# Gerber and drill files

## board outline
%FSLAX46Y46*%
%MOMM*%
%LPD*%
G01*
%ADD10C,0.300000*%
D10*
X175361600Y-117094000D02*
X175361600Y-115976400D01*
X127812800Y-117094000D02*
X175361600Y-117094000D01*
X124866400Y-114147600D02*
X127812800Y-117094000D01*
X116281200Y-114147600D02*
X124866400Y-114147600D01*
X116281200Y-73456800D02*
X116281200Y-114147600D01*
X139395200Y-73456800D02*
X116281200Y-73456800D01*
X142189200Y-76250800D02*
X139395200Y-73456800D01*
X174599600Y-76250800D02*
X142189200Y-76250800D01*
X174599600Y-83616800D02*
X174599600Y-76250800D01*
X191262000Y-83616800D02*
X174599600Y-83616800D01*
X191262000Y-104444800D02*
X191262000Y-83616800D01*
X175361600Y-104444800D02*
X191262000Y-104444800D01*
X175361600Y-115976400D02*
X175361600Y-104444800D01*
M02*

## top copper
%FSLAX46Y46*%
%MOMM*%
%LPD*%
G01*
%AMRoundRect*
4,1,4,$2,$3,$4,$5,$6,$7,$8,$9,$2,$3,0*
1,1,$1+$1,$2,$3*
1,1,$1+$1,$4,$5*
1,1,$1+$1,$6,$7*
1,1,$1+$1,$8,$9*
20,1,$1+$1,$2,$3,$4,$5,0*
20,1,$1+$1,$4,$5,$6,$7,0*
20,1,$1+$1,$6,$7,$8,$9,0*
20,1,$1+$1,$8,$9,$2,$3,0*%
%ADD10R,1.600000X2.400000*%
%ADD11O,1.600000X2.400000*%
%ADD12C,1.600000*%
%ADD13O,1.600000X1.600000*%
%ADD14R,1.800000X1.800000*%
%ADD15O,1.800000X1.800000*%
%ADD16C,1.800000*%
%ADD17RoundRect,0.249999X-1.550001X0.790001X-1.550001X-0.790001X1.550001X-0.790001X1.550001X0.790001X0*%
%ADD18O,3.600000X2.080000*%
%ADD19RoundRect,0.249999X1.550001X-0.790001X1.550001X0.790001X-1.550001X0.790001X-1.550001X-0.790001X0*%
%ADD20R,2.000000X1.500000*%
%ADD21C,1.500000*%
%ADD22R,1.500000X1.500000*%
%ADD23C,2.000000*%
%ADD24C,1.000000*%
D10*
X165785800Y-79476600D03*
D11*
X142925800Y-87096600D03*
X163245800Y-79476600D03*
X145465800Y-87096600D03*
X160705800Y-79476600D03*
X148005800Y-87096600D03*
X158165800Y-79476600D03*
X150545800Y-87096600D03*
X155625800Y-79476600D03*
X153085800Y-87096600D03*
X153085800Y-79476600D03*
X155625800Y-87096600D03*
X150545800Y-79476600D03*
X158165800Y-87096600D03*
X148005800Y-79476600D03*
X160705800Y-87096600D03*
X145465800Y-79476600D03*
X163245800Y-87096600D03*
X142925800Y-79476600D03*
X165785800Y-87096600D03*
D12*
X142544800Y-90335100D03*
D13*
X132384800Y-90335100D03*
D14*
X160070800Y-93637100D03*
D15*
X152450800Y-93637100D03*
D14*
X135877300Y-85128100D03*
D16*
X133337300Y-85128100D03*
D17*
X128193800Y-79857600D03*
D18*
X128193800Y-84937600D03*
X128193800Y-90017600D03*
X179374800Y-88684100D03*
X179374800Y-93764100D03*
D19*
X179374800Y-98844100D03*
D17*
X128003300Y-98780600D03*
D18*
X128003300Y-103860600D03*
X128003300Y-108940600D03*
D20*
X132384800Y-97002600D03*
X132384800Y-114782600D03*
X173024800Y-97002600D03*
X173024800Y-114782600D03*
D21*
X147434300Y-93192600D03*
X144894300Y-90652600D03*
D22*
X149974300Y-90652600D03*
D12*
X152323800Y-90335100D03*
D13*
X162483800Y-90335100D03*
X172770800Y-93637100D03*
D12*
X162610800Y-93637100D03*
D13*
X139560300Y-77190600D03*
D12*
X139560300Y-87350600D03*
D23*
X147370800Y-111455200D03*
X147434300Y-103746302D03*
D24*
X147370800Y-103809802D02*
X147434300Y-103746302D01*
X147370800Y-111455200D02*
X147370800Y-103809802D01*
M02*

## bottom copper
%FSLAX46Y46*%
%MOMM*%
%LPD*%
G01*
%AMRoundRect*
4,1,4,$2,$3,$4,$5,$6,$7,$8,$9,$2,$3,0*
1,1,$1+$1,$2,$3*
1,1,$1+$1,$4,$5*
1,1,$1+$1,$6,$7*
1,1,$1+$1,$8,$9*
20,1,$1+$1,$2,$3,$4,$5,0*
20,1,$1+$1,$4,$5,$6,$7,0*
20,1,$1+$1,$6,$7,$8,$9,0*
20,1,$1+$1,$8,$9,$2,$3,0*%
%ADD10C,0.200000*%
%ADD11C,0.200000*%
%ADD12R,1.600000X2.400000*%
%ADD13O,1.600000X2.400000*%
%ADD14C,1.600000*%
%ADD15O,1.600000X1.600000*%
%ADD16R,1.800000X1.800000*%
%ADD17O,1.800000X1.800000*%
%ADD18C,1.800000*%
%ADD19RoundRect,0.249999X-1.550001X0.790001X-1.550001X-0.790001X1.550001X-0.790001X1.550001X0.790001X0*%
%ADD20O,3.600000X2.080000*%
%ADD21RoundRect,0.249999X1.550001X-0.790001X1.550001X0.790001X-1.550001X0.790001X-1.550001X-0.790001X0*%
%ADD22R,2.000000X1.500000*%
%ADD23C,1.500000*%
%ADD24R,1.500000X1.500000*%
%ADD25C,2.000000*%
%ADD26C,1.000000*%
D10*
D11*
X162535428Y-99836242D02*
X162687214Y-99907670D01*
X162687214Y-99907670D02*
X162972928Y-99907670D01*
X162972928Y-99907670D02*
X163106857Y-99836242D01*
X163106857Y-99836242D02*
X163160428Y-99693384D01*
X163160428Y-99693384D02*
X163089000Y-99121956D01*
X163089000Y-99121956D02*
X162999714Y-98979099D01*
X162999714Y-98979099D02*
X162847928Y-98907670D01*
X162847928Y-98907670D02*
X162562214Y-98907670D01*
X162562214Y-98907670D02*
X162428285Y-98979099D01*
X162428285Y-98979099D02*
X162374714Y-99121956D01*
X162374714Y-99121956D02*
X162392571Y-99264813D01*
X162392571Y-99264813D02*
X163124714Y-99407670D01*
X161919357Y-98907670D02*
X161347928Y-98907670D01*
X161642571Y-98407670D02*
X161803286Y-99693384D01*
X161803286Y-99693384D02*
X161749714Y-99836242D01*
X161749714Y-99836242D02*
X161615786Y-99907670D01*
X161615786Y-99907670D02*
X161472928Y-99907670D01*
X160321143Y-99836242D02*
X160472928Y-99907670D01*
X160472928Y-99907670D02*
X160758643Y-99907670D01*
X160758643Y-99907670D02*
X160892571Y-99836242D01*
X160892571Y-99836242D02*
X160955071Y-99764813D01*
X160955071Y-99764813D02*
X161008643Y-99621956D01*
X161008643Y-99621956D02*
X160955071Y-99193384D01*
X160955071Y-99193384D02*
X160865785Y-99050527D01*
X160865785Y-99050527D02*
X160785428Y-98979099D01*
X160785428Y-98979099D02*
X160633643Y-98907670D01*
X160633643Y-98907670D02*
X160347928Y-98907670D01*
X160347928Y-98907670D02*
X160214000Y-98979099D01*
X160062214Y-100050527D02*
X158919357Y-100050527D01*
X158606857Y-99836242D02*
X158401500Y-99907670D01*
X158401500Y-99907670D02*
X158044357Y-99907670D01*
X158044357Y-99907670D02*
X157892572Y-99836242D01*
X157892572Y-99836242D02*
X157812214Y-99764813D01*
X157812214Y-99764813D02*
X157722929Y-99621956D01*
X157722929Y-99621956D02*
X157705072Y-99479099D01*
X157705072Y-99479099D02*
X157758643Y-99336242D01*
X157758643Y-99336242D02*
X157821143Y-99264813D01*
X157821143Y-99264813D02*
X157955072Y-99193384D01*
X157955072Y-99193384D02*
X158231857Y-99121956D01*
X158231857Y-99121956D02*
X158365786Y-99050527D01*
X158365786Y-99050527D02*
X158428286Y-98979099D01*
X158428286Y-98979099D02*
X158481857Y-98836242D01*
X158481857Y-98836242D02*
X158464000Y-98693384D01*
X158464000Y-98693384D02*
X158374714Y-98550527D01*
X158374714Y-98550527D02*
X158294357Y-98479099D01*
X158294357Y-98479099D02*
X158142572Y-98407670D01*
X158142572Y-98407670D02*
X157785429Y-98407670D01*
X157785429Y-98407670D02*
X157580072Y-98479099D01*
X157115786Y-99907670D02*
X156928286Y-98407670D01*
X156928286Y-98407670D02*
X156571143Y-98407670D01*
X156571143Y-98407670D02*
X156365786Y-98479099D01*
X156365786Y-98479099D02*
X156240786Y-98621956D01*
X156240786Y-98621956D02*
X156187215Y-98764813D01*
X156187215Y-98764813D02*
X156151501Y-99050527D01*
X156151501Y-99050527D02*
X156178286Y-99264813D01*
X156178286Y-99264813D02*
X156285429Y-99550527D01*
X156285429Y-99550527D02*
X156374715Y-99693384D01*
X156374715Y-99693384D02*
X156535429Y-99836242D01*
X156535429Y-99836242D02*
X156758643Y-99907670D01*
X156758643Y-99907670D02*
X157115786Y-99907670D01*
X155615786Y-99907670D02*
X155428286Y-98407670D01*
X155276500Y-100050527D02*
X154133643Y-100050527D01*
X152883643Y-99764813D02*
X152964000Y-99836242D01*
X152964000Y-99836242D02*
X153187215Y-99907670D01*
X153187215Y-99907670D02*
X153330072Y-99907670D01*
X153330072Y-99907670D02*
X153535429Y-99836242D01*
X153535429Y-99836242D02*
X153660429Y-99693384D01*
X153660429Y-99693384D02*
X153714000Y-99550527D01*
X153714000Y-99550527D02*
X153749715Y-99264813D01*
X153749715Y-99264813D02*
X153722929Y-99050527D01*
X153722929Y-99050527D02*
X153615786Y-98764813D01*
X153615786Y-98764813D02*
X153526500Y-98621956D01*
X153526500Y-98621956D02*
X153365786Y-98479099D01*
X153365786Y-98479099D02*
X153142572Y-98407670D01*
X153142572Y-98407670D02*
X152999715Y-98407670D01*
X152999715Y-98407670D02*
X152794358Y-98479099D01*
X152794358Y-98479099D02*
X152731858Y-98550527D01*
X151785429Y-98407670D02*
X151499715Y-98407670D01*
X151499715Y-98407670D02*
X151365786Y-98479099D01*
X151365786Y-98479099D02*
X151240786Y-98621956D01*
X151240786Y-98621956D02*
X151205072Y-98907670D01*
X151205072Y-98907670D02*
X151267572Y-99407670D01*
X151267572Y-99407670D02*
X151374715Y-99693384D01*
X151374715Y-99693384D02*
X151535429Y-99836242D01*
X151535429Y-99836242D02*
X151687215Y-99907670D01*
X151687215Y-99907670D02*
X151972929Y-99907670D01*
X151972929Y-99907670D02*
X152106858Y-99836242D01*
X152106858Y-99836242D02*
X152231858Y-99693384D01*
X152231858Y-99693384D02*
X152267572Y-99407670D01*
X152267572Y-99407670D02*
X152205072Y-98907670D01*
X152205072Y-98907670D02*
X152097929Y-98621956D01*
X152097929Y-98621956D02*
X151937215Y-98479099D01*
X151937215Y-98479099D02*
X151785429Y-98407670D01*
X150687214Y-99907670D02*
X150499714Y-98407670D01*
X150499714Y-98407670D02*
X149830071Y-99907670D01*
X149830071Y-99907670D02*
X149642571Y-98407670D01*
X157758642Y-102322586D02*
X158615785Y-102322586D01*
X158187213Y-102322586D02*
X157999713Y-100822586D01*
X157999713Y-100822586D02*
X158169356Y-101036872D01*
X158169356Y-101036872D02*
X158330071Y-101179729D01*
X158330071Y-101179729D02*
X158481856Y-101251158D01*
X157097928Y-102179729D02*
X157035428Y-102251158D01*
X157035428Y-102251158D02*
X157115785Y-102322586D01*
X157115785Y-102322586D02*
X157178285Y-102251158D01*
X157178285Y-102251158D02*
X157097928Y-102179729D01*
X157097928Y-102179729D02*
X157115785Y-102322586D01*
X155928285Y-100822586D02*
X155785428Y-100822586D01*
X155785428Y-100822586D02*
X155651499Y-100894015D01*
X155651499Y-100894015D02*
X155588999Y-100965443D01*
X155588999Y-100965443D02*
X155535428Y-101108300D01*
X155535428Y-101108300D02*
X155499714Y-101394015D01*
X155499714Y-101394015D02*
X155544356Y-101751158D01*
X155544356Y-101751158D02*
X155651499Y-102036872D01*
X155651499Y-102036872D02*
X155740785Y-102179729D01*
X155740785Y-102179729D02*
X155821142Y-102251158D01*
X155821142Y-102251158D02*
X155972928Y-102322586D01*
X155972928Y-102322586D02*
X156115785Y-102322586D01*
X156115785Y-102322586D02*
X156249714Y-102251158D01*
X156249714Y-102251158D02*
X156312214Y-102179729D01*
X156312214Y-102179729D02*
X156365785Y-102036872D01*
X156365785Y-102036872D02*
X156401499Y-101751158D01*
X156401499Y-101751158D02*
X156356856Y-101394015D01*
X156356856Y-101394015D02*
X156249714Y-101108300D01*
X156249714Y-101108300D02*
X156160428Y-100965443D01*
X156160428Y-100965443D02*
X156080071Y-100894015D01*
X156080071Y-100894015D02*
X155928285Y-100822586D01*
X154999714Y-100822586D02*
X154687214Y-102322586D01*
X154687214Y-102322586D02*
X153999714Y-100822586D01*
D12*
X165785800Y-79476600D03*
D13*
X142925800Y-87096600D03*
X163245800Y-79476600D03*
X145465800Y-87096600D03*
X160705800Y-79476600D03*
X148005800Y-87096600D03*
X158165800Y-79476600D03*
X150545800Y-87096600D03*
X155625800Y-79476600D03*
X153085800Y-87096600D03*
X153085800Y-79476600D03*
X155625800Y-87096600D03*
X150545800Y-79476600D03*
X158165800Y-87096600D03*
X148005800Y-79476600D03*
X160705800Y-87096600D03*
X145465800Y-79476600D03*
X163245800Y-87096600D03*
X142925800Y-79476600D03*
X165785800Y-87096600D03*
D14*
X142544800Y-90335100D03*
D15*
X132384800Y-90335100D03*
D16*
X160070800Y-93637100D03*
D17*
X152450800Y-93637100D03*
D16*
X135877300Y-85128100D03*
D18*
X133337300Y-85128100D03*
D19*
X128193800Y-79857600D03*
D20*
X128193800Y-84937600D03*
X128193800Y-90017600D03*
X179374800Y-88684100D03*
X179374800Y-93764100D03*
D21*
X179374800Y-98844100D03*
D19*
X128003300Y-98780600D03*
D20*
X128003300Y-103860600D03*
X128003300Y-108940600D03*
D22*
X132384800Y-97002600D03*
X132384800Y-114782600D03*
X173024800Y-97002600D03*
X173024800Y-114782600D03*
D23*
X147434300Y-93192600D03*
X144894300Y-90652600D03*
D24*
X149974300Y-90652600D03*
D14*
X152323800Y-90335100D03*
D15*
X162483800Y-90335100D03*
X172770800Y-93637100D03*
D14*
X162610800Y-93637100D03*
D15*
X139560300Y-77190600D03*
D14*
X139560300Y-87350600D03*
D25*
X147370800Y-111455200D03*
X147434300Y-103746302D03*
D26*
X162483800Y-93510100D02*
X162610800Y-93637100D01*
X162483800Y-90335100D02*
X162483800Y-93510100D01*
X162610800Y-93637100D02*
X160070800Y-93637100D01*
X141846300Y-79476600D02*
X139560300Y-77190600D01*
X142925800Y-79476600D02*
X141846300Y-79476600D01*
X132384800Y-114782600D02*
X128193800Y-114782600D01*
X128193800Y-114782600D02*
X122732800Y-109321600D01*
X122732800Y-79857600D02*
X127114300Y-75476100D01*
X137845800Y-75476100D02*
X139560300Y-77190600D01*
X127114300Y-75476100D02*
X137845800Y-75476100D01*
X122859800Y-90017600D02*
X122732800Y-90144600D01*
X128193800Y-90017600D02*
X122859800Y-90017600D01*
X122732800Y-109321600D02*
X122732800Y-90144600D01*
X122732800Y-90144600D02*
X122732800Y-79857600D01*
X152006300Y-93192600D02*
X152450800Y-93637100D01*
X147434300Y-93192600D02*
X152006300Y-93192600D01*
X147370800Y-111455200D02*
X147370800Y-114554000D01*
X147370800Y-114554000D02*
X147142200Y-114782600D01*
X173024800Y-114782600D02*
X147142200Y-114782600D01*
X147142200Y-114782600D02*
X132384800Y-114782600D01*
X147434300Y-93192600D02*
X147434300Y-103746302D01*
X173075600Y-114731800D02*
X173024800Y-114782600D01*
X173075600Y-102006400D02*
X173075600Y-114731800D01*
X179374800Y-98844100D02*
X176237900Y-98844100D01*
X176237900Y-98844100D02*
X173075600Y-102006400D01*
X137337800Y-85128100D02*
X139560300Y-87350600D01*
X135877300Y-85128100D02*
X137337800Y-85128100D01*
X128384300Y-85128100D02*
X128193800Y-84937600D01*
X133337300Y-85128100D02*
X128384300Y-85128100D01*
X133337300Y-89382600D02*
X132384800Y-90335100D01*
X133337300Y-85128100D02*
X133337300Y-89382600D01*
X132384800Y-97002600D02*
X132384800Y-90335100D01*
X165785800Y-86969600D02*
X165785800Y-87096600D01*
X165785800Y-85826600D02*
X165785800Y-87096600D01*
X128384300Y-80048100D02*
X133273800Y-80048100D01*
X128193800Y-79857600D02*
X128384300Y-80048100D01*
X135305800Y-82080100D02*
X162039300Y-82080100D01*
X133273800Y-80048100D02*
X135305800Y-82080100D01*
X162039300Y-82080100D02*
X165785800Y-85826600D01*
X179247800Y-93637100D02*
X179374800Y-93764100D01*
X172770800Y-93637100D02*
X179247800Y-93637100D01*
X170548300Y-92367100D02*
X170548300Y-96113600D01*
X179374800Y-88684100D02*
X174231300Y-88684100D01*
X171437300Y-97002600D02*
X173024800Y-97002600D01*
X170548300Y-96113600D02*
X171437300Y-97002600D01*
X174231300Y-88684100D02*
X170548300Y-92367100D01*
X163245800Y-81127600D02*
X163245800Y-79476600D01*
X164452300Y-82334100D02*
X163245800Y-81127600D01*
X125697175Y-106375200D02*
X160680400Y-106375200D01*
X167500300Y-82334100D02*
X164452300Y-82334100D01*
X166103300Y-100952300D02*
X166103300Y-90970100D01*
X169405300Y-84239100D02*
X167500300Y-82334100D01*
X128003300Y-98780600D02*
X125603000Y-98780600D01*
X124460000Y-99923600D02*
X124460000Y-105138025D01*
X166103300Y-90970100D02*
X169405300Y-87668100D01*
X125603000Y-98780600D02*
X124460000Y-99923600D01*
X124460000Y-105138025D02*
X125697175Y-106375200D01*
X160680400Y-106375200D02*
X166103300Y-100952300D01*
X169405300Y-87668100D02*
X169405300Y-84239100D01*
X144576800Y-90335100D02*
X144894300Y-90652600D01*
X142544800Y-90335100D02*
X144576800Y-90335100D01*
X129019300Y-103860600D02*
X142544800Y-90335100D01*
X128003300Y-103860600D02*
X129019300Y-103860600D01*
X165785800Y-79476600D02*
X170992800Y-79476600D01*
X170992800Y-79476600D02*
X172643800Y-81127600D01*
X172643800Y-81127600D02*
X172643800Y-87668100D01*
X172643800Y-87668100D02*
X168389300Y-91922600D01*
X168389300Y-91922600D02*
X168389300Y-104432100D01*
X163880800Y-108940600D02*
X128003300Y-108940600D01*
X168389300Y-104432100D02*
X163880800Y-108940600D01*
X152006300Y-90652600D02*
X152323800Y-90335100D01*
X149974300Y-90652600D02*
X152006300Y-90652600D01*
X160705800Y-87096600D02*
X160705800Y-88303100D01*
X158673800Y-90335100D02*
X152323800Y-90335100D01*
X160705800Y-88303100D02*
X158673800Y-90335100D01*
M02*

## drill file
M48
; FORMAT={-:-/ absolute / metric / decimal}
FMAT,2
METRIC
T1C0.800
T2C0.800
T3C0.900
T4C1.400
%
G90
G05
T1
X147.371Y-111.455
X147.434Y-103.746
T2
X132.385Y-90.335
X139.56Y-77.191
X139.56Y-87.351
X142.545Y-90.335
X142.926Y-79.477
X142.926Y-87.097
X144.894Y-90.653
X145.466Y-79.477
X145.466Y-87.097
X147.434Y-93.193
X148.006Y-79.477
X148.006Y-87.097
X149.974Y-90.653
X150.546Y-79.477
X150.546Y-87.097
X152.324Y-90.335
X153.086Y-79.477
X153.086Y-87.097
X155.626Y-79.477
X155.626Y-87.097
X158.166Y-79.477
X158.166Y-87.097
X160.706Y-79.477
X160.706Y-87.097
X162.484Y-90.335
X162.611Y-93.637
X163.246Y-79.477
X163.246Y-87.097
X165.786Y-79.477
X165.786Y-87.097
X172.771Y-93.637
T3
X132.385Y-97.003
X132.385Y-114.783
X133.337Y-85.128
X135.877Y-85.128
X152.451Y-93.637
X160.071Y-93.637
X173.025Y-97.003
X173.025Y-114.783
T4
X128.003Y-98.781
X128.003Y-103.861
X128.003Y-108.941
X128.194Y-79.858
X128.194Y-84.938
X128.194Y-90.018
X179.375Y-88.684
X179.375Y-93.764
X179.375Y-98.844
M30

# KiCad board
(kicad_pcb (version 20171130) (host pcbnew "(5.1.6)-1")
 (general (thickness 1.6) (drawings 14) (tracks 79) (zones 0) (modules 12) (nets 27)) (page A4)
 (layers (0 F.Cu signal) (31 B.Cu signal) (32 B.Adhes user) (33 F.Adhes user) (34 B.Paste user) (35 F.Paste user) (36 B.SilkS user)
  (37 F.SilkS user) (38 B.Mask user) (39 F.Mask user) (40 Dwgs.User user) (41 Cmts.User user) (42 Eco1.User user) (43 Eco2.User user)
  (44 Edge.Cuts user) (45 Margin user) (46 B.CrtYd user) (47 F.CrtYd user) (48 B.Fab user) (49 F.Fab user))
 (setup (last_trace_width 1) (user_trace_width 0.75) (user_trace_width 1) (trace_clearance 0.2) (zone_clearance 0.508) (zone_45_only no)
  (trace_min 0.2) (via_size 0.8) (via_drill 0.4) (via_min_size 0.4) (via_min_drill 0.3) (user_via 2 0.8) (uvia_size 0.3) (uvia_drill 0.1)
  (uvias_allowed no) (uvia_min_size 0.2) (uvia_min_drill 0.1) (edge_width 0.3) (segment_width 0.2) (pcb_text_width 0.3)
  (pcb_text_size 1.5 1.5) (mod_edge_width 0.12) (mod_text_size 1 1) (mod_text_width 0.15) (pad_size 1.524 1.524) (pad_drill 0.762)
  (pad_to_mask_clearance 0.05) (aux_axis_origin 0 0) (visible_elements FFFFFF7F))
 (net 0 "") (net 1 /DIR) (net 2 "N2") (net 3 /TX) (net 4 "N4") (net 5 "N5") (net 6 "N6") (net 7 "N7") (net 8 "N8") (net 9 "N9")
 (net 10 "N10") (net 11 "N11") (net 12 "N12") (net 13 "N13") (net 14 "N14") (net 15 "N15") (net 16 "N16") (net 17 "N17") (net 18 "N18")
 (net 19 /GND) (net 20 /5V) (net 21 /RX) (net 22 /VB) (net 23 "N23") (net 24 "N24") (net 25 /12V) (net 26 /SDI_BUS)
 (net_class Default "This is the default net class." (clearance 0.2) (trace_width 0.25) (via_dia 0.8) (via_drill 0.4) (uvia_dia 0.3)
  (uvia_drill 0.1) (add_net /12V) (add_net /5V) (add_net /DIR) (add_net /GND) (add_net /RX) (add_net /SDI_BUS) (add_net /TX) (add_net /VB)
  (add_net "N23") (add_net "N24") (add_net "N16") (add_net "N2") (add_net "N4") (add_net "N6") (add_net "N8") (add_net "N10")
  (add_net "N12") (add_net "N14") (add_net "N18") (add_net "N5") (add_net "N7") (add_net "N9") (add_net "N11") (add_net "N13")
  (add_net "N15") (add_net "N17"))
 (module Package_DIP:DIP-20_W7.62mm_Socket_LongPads (layer F.Cu) (at 165.7858 79.4766 270)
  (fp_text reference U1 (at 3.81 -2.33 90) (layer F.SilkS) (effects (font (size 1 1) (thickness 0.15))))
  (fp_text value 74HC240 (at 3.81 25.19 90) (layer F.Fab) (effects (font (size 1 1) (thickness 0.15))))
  (pad 1 thru_hole rect (at 0 0 270) (size 2.4 1.6) (drill 0.8) (layers *.Cu *.Mask) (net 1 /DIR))
  (pad 11 thru_hole oval (at 7.62 22.86 270) (size 2.4 1.6) (drill 0.8) (layers *.Cu *.Mask) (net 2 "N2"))
  (pad 2 thru_hole oval (at 0 2.54 270) (size 2.4 1.6) (drill 0.8) (layers *.Cu *.Mask) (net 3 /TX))
  (pad 12 thru_hole oval (at 7.62 20.32 270) (size 2.4 1.6) (drill 0.8) (layers *.Cu *.Mask) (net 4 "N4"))
  (pad 3 thru_hole oval (at 0 5.08 270) (size 2.4 1.6) (drill 0.8) (layers *.Cu *.Mask) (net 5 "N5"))
  (pad 13 thru_hole oval (at 7.62 17.78 270) (size 2.4 1.6) (drill 0.8) (layers *.Cu *.Mask) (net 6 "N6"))
  (pad 4 thru_hole oval (at 0 7.62 270) (size 2.4 1.6) (drill 0.8) (layers *.Cu *.Mask) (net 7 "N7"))
  (pad 14 thru_hole oval (at 7.62 15.24 270) (size 2.4 1.6) (drill 0.8) (layers *.Cu *.Mask) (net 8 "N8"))
  (pad 5 thru_hole oval (at 0 10.16 270) (size 2.4 1.6) (drill 0.8) (layers *.Cu *.Mask) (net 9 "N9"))
  (pad 15 thru_hole oval (at 7.62 12.7 270) (size 2.4 1.6) (drill 0.8) (layers *.Cu *.Mask) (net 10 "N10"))
  (pad 6 thru_hole oval (at 0 12.7 270) (size 2.4 1.6) (drill 0.8) (layers *.Cu *.Mask) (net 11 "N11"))
  (pad 16 thru_hole oval (at 7.62 10.16 270) (size 2.4 1.6) (drill 0.8) (layers *.Cu *.Mask) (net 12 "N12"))
  (pad 7 thru_hole oval (at 0 15.24 270) (size 2.4 1.6) (drill 0.8) (layers *.Cu *.Mask) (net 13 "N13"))
  (pad 17 thru_hole oval (at 7.62 7.62 270) (size 2.4 1.6) (drill 0.8) (layers *.Cu *.Mask) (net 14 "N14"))
  (pad 8 thru_hole oval (at 0 17.78 270) (size 2.4 1.6) (drill 0.8) (layers *.Cu *.Mask) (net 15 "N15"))
  (pad 18 thru_hole oval (at 7.62 5.08 270) (size 2.4 1.6) (drill 0.8) (layers *.Cu *.Mask) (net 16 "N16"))
  (pad 9 thru_hole oval (at 0 20.32 270) (size 2.4 1.6) (drill 0.8) (layers *.Cu *.Mask) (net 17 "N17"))
  (pad 19 thru_hole oval (at 7.62 2.54 270) (size 2.4 1.6) (drill 0.8) (layers *.Cu *.Mask) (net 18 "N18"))
  (pad 10 thru_hole oval (at 0 22.86 270) (size 2.4 1.6) (drill 0.8) (layers *.Cu *.Mask) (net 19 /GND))
  (pad 20 thru_hole oval (at 7.62 0 270) (size 2.4 1.6) (drill 0.8) (layers *.Cu *.Mask) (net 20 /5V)))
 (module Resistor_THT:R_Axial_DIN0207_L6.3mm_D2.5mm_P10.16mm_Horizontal (layer F.Cu) (at 142.5448 90.3351 180)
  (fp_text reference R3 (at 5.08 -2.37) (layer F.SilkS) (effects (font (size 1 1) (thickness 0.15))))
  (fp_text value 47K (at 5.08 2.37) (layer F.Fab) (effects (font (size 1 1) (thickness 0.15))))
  (pad 1 thru_hole circle (at 0 0 180) (size 1.6 1.6) (drill 0.8) (layers *.Cu *.Mask) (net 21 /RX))
  (pad 2 thru_hole oval (at 10.16 0 180) (size 1.6 1.6) (drill 0.8) (layers *.Cu *.Mask) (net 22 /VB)))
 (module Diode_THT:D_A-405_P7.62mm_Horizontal (layer F.Cu) (at 160.0708 93.6371 180)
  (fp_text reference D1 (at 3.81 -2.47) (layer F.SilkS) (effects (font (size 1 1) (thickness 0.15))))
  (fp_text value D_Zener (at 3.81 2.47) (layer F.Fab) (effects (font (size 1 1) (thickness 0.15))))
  (pad 1 thru_hole rect (at 0 0 180) (size 1.8 1.8) (drill 0.9) (layers *.Cu *.Mask) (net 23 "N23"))
  (pad 2 thru_hole oval (at 7.62 0 180) (size 1.8 1.8) (drill 0.9) (layers *.Cu *.Mask) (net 19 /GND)))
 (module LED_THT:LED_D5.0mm (layer F.Cu) (at 135.8773 85.1281 180)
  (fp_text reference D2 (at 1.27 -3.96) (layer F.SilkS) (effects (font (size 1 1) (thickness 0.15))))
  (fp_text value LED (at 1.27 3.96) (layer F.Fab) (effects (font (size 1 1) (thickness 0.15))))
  (pad 1 thru_hole rect (at 0 0 180) (size 1.8 1.8) (drill 0.9) (layers *.Cu *.Mask) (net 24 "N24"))
  (pad 2 thru_hole circle (at 2.54 0 180) (size 1.8 1.8) (drill 0.9) (layers *.Cu *.Mask) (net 22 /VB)))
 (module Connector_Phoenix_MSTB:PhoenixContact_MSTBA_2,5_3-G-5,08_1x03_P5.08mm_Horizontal (layer F.Cu) (at 128.1938 79.8576 270)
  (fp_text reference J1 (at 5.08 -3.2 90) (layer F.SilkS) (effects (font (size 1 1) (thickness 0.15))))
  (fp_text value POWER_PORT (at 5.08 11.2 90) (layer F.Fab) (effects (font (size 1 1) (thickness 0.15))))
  (pad 1 thru_hole roundrect (at 0 0 270) (size 2.08 3.6) (drill 1.4) (layers *.Cu *.Mask) (roundrect_rratio 0.120192) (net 20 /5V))
  (pad 2 thru_hole oval (at 5.08 0 270) (size 2.08 3.6) (drill 1.4) (layers *.Cu *.Mask) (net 22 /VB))
  (pad 3 thru_hole oval (at 10.16 0 270) (size 2.08 3.6) (drill 1.4) (layers *.Cu *.Mask) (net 19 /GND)))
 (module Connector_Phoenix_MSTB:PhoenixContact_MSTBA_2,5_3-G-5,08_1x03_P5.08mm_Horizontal (layer F.Cu) (at 179.3748 98.8441 90)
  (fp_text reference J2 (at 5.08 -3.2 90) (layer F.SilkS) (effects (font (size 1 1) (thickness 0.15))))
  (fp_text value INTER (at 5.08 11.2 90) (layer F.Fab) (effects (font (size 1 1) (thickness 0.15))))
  (pad 3 thru_hole oval (at 10.16 0 90) (size 2.08 3.6) (drill 1.4) (layers *.Cu *.Mask) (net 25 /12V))
  (pad 2 thru_hole oval (at 5.08 0 90) (size 2.08 3.6) (drill 1.4) (layers *.Cu *.Mask) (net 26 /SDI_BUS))
  (pad 1 thru_hole roundrect (at 0 0 90) (size 2.08 3.6) (drill 1.4) (layers *.Cu *.Mask) (roundrect_rratio 0.120192) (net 19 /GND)))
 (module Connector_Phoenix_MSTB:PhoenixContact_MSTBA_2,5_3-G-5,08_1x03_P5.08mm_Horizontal (layer F.Cu) (at 128.0033 98.7806 270)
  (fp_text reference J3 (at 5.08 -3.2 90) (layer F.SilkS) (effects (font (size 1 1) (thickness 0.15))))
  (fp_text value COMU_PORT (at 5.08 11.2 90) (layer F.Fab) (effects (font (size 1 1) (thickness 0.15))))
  (pad 1 thru_hole roundrect (at 0 0 270) (size 2.08 3.6) (drill 1.4) (layers *.Cu *.Mask) (roundrect_rratio 0.120192) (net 3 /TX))
  (pad 2 thru_hole oval (at 5.08 0 270) (size 2.08 3.6) (drill 1.4) (layers *.Cu *.Mask) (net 21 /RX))
  (pad 3 thru_hole oval (at 10.16 0 270) (size 2.08 3.6) (drill 1.4) (layers *.Cu *.Mask) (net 1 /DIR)))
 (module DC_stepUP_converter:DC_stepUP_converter (layer F.Cu) (at 152.7048 90.6526)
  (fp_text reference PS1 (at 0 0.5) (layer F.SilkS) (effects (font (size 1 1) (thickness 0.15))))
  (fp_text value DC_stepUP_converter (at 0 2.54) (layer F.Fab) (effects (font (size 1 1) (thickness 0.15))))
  (pad 1 thru_hole rect (at -20.32 6.35) (size 2 1.5) (drill 0.9) (layers *.Cu *.Mask) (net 22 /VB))
  (pad 2 thru_hole rect (at -20.32 24.13) (size 2 1.5) (drill 0.9) (layers *.Cu *.Mask) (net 19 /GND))
  (pad 3 thru_hole rect (at 20.32 6.35) (size 2 1.5) (drill 0.9) (layers *.Cu *.Mask) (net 25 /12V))
  (pad 4 thru_hole rect (at 20.32 24.13) (size 2 1.5) (drill 0.9) (layers *.Cu *.Mask) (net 19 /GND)))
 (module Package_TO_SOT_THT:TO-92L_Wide (layer F.Cu) (at 149.9743 90.6526 180)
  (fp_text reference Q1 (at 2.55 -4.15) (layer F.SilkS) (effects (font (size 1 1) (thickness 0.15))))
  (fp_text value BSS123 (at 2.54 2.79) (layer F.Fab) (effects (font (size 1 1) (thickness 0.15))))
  (pad 2 thru_hole circle (at 2.54 -2.54 270) (size 1.5 1.5) (drill 0.8) (layers *.Cu *.Mask) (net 19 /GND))
  (pad 3 thru_hole circle (at 5.08 0 270) (size 1.5 1.5) (drill 0.8) (layers *.Cu *.Mask) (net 21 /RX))
  (pad 1 thru_hole rect (at 0 0 270) (size 1.5 1.5) (drill 0.8) (layers *.Cu *.Mask) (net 16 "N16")))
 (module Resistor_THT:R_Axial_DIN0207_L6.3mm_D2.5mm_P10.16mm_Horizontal (layer F.Cu) (at 152.3238 90.3351)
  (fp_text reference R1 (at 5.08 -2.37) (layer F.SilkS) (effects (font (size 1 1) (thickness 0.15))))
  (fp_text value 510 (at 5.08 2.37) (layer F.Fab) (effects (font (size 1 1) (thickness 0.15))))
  (pad 1 thru_hole circle (at 0 0) (size 1.6 1.6) (drill 0.8) (layers *.Cu *.Mask) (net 16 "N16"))
  (pad 2 thru_hole oval (at 10.16 0) (size 1.6 1.6) (drill 0.8) (layers *.Cu *.Mask) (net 23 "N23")))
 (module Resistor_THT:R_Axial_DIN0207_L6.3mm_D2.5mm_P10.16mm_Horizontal (layer F.Cu) (at 162.6108 93.6371)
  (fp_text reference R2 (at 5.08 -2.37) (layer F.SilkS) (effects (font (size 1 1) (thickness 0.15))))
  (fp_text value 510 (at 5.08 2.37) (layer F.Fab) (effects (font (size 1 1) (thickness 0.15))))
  (pad 2 thru_hole oval (at 10.16 0) (size 1.6 1.6) (drill 0.8) (layers *.Cu *.Mask) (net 26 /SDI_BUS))
  (pad 1 thru_hole circle (at 0 0) (size 1.6 1.6) (drill 0.8) (layers *.Cu *.Mask) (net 23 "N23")))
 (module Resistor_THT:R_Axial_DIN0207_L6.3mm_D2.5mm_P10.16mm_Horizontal (layer F.Cu) (at 139.5603 87.3506 90)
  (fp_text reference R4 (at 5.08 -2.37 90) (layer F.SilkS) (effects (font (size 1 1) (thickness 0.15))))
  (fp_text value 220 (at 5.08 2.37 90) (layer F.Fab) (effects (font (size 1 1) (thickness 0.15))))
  (pad 2 thru_hole oval (at 10.16 0 90) (size 1.6 1.6) (drill 0.8) (layers *.Cu *.Mask) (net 19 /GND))
  (pad 1 thru_hole circle (at 0 0 90) (size 1.6 1.6) (drill 0.8) (layers *.Cu *.Mask) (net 24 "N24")))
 (gr_line (start 175.3616 117.094) (end 175.3616 115.9764) (layer Edge.Cuts) (width 0.3))
 (gr_line (start 127.8128 117.094) (end 175.3616 117.094) (layer Edge.Cuts) (width 0.3))
 (gr_line (start 124.8664 114.1476) (end 127.8128 117.094) (layer Edge.Cuts) (width 0.3))
 (gr_line (start 116.2812 114.1476) (end 124.8664 114.1476) (layer Edge.Cuts) (width 0.3))
 (gr_line (start 116.2812 73.4568) (end 116.2812 114.1476) (layer Edge.Cuts) (width 0.3))
 (gr_line (start 139.3952 73.4568) (end 116.2812 73.4568) (layer Edge.Cuts) (width 0.3))
 (gr_line (start 142.1892 76.2508) (end 139.3952 73.4568) (layer Edge.Cuts) (width 0.3))
 (gr_line (start 174.5996 76.2508) (end 142.1892 76.2508) (layer Edge.Cuts) (width 0.3))
 (gr_line (start 174.5996 83.6168) (end 174.5996 76.2508) (layer Edge.Cuts) (width 0.3))
 (gr_line (start 191.262 83.6168) (end 174.5996 83.6168) (layer Edge.Cuts) (width 0.3))
 (gr_line (start 191.262 104.4448) (end 191.262 83.6168) (layer Edge.Cuts) (width 0.3))
 (gr_line (start 175.3616 104.4448) (end 191.262 104.4448) (layer Edge.Cuts) (width 0.3))
 (gr_line (start 175.3616 115.9764) (end 175.3616 104.4448) (layer Edge.Cuts) (width 0.3))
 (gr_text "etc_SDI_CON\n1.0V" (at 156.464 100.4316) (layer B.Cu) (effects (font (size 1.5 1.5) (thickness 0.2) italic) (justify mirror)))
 (segment (start 162.4838 93.5101) (end 162.6108 93.6371) (width 1) (layer B.Cu) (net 23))
 (segment (start 162.4838 90.3351) (end 162.4838 93.5101) (width 1) (layer B.Cu) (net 23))
 (segment (start 162.6108 93.6371) (end 160.0708 93.6371) (width 1) (layer B.Cu) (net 23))
 (segment (start 141.8463 79.4766) (end 139.5603 77.1906) (width 1) (layer B.Cu) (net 19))
 (segment (start 142.9258 79.4766) (end 141.8463 79.4766) (width 1) (layer B.Cu) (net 19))
 (segment (start 132.3848 114.7826) (end 128.1938 114.7826) (width 1) (layer B.Cu) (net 19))
 (segment (start 128.1938 114.7826) (end 122.7328 109.3216) (width 1) (layer B.Cu) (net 19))
 (segment (start 122.7328 79.8576) (end 127.1143 75.4761) (width 1) (layer B.Cu) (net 19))
 (segment (start 137.8458 75.4761) (end 139.5603 77.1906) (width 1) (layer B.Cu) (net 19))
 (segment (start 127.1143 75.4761) (end 137.8458 75.4761) (width 1) (layer B.Cu) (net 19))
 (segment (start 122.8598 90.0176) (end 122.7328 90.1446) (width 1) (layer B.Cu) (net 19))
 (segment (start 128.1938 90.0176) (end 122.8598 90.0176) (width 1) (layer B.Cu) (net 19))
 (segment (start 122.7328 109.3216) (end 122.7328 90.1446) (width 1) (layer B.Cu) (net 19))
 (segment (start 122.7328 90.1446) (end 122.7328 79.8576) (width 1) (layer B.Cu) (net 19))
 (segment (start 152.0063 93.1926) (end 152.4508 93.6371) (width 1) (layer B.Cu) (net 19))
 (segment (start 147.4343 93.1926) (end 152.0063 93.1926) (width 1) (layer B.Cu) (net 19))
 (via (at 147.3708 111.4552) (size 2) (drill 0.8) (layers F.Cu B.Cu) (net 19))
 (segment (start 147.3708 111.4552) (end 147.3708 114.554) (width 1) (layer B.Cu) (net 19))
 (segment (start 147.3708 114.554) (end 147.1422 114.7826) (width 1) (layer B.Cu) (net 19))
 (segment (start 173.0248 114.7826) (end 147.1422 114.7826) (width 1) (layer B.Cu) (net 19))
 (segment (start 147.1422 114.7826) (end 132.3848 114.7826) (width 1) (layer B.Cu) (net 19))
 (via (at 147.4343 103.746302) (size 2) (drill 0.8) (layers F.Cu B.Cu) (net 19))
 (segment (start 147.4343 93.1926) (end 147.4343 103.746302) (width 1) (layer B.Cu) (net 19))
 (segment (start 147.3708 103.809802) (end 147.4343 103.746302) (width 1) (layer F.Cu) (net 19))
 (segment (start 147.3708 111.4552) (end 147.3708 103.809802) (width 1) (layer F.Cu) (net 19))
 (segment (start 173.0756 114.7318) (end 173.0248 114.7826) (width 1) (layer B.Cu) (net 19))
 (segment (start 173.0756 102.0064) (end 173.0756 114.7318) (width 1) (layer B.Cu) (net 19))
 (segment (start 179.3748 98.8441) (end 176.2379 98.8441) (width 1) (layer B.Cu) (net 19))
 (segment (start 176.2379 98.8441) (end 173.0756 102.0064) (width 1) (layer B.Cu) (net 19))
 (segment (start 137.3378 85.1281) (end 139.5603 87.3506) (width 1) (layer B.Cu) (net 24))
 (segment (start 135.8773 85.1281) (end 137.3378 85.1281) (width 1) (layer B.Cu) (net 24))
 (segment (start 128.3843 85.1281) (end 128.1938 84.9376) (width 1) (layer B.Cu) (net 22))
 (segment (start 133.3373 85.1281) (end 128.3843 85.1281) (width 1) (layer B.Cu) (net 22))
 (segment (start 133.3373 89.3826) (end 132.3848 90.3351) (width 1) (layer B.Cu) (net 22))
 (segment (start 133.3373 85.1281) (end 133.3373 89.3826) (width 1) (layer B.Cu) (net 22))
 (segment (start 132.3848 97.0026) (end 132.3848 90.3351) (width 1) (layer B.Cu) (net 22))
 (segment (start 165.7858 86.9696) (end 165.7858 87.0966) (width 1) (layer B.Cu) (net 20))
 (segment (start 165.7858 85.8266) (end 165.7858 87.0966) (width 1) (layer B.Cu) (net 20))
 (segment (start 128.3843 80.0481) (end 133.2738 80.0481) (width 1) (layer B.Cu) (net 20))
 (segment (start 128.1938 79.8576) (end 128.3843 80.0481) (width 1) (layer B.Cu) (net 20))
 (segment (start 135.3058 82.0801) (end 162.0393 82.0801) (width 1) (layer B.Cu) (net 20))
 (segment (start 133.2738 80.0481) (end 135.3058 82.0801) (width 1) (layer B.Cu) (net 20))
 (segment (start 162.0393 82.0801) (end 165.7858 85.8266) (width 1) (layer B.Cu) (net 20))
 (segment (start 179.2478 93.6371) (end 179.3748 93.7641) (width 1) (layer B.Cu) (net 26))
 (segment (start 172.7708 93.6371) (end 179.2478 93.6371) (width 1) (layer B.Cu) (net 26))
 (segment (start 170.5483 92.3671) (end 170.5483 96.1136) (width 1) (layer B.Cu) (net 25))
 (segment (start 179.3748 88.6841) (end 174.2313 88.6841) (width 1) (layer B.Cu) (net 25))
 (segment (start 171.4373 97.0026) (end 173.0248 97.0026) (width 1) (layer B.Cu) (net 25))
 (segment (start 170.5483 96.1136) (end 171.4373 97.0026) (width 1) (layer B.Cu) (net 25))
 (segment (start 174.2313 88.6841) (end 170.5483 92.3671) (width 1) (layer B.Cu) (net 25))
 (segment (start 163.2458 81.1276) (end 163.2458 79.4766) (width 1) (layer B.Cu) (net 3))
 (segment (start 164.4523 82.3341) (end 163.2458 81.1276) (width 1) (layer B.Cu) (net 3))
 (segment (start 125.697175 106.3752) (end 160.6804 106.3752) (width 1) (layer B.Cu) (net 3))
 (segment (start 167.5003 82.3341) (end 164.4523 82.3341) (width 1) (layer B.Cu) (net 3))
 (segment (start 166.1033 100.9523) (end 166.1033 90.9701) (width 1) (layer B.Cu) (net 3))
 (segment (start 169.4053 84.2391) (end 167.5003 82.3341) (width 1) (layer B.Cu) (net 3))
 (segment (start 128.0033 98.7806) (end 125.603 98.7806) (width 1) (layer B.Cu) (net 3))
 (segment (start 124.46 99.9236) (end 124.46 105.138025) (width 1) (layer B.Cu) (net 3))
 (segment (start 166.1033 90.9701) (end 169.4053 87.6681) (width 1) (layer B.Cu) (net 3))
 (segment (start 125.603 98.7806) (end 124.46 99.9236) (width 1) (layer B.Cu) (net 3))
 (segment (start 124.46 105.138025) (end 125.697175 106.3752) (width 1) (layer B.Cu) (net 3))
 (segment (start 160.6804 106.3752) (end 166.1033 100.9523) (width 1) (layer B.Cu) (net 3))
 (segment (start 169.4053 87.6681) (end 169.4053 84.2391) (width 1) (layer B.Cu) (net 3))
 (segment (start 144.5768 90.3351) (end 144.8943 90.6526) (width 1) (layer B.Cu) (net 21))
 (segment (start 142.5448 90.3351) (end 144.5768 90.3351) (width 1) (layer B.Cu) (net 21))
 (segment (start 129.0193 103.8606) (end 142.5448 90.3351) (width 1) (layer B.Cu) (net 21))
 (segment (start 128.0033 103.8606) (end 129.0193 103.8606) (width 1) (layer B.Cu) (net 21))
 (segment (start 165.7858 79.4766) (end 170.9928 79.4766) (width 1) (layer B.Cu) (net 1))
 (segment (start 170.9928 79.4766) (end 172.6438 81.1276) (width 1) (layer B.Cu) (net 1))
 (segment (start 172.6438 81.1276) (end 172.6438 87.6681) (width 1) (layer B.Cu) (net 1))
 (segment (start 172.6438 87.6681) (end 168.3893 91.9226) (width 1) (layer B.Cu) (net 1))
 (segment (start 168.3893 91.9226) (end 168.3893 104.4321) (width 1) (layer B.Cu) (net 1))
 (segment (start 163.8808 108.9406) (end 128.0033 108.9406) (width 1) (layer B.Cu) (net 1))
 (segment (start 168.3893 104.4321) (end 163.8808 108.9406) (width 1) (layer B.Cu) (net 1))
 (segment (start 152.0063 90.6526) (end 152.3238 90.3351) (width 1) (layer B.Cu) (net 16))
 (segment (start 149.9743 90.6526) (end 152.0063 90.6526) (width 1) (layer B.Cu) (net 16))
 (segment (start 160.7058 87.0966) (end 160.7058 88.3031) (width 1) (layer B.Cu) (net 16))
 (segment (start 158.6738 90.3351) (end 152.3238 90.3351) (width 1) (layer B.Cu) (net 16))
 (segment (start 160.7058 88.3031) (end 158.6738 90.3351) (width 1) (layer B.Cu) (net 16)))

